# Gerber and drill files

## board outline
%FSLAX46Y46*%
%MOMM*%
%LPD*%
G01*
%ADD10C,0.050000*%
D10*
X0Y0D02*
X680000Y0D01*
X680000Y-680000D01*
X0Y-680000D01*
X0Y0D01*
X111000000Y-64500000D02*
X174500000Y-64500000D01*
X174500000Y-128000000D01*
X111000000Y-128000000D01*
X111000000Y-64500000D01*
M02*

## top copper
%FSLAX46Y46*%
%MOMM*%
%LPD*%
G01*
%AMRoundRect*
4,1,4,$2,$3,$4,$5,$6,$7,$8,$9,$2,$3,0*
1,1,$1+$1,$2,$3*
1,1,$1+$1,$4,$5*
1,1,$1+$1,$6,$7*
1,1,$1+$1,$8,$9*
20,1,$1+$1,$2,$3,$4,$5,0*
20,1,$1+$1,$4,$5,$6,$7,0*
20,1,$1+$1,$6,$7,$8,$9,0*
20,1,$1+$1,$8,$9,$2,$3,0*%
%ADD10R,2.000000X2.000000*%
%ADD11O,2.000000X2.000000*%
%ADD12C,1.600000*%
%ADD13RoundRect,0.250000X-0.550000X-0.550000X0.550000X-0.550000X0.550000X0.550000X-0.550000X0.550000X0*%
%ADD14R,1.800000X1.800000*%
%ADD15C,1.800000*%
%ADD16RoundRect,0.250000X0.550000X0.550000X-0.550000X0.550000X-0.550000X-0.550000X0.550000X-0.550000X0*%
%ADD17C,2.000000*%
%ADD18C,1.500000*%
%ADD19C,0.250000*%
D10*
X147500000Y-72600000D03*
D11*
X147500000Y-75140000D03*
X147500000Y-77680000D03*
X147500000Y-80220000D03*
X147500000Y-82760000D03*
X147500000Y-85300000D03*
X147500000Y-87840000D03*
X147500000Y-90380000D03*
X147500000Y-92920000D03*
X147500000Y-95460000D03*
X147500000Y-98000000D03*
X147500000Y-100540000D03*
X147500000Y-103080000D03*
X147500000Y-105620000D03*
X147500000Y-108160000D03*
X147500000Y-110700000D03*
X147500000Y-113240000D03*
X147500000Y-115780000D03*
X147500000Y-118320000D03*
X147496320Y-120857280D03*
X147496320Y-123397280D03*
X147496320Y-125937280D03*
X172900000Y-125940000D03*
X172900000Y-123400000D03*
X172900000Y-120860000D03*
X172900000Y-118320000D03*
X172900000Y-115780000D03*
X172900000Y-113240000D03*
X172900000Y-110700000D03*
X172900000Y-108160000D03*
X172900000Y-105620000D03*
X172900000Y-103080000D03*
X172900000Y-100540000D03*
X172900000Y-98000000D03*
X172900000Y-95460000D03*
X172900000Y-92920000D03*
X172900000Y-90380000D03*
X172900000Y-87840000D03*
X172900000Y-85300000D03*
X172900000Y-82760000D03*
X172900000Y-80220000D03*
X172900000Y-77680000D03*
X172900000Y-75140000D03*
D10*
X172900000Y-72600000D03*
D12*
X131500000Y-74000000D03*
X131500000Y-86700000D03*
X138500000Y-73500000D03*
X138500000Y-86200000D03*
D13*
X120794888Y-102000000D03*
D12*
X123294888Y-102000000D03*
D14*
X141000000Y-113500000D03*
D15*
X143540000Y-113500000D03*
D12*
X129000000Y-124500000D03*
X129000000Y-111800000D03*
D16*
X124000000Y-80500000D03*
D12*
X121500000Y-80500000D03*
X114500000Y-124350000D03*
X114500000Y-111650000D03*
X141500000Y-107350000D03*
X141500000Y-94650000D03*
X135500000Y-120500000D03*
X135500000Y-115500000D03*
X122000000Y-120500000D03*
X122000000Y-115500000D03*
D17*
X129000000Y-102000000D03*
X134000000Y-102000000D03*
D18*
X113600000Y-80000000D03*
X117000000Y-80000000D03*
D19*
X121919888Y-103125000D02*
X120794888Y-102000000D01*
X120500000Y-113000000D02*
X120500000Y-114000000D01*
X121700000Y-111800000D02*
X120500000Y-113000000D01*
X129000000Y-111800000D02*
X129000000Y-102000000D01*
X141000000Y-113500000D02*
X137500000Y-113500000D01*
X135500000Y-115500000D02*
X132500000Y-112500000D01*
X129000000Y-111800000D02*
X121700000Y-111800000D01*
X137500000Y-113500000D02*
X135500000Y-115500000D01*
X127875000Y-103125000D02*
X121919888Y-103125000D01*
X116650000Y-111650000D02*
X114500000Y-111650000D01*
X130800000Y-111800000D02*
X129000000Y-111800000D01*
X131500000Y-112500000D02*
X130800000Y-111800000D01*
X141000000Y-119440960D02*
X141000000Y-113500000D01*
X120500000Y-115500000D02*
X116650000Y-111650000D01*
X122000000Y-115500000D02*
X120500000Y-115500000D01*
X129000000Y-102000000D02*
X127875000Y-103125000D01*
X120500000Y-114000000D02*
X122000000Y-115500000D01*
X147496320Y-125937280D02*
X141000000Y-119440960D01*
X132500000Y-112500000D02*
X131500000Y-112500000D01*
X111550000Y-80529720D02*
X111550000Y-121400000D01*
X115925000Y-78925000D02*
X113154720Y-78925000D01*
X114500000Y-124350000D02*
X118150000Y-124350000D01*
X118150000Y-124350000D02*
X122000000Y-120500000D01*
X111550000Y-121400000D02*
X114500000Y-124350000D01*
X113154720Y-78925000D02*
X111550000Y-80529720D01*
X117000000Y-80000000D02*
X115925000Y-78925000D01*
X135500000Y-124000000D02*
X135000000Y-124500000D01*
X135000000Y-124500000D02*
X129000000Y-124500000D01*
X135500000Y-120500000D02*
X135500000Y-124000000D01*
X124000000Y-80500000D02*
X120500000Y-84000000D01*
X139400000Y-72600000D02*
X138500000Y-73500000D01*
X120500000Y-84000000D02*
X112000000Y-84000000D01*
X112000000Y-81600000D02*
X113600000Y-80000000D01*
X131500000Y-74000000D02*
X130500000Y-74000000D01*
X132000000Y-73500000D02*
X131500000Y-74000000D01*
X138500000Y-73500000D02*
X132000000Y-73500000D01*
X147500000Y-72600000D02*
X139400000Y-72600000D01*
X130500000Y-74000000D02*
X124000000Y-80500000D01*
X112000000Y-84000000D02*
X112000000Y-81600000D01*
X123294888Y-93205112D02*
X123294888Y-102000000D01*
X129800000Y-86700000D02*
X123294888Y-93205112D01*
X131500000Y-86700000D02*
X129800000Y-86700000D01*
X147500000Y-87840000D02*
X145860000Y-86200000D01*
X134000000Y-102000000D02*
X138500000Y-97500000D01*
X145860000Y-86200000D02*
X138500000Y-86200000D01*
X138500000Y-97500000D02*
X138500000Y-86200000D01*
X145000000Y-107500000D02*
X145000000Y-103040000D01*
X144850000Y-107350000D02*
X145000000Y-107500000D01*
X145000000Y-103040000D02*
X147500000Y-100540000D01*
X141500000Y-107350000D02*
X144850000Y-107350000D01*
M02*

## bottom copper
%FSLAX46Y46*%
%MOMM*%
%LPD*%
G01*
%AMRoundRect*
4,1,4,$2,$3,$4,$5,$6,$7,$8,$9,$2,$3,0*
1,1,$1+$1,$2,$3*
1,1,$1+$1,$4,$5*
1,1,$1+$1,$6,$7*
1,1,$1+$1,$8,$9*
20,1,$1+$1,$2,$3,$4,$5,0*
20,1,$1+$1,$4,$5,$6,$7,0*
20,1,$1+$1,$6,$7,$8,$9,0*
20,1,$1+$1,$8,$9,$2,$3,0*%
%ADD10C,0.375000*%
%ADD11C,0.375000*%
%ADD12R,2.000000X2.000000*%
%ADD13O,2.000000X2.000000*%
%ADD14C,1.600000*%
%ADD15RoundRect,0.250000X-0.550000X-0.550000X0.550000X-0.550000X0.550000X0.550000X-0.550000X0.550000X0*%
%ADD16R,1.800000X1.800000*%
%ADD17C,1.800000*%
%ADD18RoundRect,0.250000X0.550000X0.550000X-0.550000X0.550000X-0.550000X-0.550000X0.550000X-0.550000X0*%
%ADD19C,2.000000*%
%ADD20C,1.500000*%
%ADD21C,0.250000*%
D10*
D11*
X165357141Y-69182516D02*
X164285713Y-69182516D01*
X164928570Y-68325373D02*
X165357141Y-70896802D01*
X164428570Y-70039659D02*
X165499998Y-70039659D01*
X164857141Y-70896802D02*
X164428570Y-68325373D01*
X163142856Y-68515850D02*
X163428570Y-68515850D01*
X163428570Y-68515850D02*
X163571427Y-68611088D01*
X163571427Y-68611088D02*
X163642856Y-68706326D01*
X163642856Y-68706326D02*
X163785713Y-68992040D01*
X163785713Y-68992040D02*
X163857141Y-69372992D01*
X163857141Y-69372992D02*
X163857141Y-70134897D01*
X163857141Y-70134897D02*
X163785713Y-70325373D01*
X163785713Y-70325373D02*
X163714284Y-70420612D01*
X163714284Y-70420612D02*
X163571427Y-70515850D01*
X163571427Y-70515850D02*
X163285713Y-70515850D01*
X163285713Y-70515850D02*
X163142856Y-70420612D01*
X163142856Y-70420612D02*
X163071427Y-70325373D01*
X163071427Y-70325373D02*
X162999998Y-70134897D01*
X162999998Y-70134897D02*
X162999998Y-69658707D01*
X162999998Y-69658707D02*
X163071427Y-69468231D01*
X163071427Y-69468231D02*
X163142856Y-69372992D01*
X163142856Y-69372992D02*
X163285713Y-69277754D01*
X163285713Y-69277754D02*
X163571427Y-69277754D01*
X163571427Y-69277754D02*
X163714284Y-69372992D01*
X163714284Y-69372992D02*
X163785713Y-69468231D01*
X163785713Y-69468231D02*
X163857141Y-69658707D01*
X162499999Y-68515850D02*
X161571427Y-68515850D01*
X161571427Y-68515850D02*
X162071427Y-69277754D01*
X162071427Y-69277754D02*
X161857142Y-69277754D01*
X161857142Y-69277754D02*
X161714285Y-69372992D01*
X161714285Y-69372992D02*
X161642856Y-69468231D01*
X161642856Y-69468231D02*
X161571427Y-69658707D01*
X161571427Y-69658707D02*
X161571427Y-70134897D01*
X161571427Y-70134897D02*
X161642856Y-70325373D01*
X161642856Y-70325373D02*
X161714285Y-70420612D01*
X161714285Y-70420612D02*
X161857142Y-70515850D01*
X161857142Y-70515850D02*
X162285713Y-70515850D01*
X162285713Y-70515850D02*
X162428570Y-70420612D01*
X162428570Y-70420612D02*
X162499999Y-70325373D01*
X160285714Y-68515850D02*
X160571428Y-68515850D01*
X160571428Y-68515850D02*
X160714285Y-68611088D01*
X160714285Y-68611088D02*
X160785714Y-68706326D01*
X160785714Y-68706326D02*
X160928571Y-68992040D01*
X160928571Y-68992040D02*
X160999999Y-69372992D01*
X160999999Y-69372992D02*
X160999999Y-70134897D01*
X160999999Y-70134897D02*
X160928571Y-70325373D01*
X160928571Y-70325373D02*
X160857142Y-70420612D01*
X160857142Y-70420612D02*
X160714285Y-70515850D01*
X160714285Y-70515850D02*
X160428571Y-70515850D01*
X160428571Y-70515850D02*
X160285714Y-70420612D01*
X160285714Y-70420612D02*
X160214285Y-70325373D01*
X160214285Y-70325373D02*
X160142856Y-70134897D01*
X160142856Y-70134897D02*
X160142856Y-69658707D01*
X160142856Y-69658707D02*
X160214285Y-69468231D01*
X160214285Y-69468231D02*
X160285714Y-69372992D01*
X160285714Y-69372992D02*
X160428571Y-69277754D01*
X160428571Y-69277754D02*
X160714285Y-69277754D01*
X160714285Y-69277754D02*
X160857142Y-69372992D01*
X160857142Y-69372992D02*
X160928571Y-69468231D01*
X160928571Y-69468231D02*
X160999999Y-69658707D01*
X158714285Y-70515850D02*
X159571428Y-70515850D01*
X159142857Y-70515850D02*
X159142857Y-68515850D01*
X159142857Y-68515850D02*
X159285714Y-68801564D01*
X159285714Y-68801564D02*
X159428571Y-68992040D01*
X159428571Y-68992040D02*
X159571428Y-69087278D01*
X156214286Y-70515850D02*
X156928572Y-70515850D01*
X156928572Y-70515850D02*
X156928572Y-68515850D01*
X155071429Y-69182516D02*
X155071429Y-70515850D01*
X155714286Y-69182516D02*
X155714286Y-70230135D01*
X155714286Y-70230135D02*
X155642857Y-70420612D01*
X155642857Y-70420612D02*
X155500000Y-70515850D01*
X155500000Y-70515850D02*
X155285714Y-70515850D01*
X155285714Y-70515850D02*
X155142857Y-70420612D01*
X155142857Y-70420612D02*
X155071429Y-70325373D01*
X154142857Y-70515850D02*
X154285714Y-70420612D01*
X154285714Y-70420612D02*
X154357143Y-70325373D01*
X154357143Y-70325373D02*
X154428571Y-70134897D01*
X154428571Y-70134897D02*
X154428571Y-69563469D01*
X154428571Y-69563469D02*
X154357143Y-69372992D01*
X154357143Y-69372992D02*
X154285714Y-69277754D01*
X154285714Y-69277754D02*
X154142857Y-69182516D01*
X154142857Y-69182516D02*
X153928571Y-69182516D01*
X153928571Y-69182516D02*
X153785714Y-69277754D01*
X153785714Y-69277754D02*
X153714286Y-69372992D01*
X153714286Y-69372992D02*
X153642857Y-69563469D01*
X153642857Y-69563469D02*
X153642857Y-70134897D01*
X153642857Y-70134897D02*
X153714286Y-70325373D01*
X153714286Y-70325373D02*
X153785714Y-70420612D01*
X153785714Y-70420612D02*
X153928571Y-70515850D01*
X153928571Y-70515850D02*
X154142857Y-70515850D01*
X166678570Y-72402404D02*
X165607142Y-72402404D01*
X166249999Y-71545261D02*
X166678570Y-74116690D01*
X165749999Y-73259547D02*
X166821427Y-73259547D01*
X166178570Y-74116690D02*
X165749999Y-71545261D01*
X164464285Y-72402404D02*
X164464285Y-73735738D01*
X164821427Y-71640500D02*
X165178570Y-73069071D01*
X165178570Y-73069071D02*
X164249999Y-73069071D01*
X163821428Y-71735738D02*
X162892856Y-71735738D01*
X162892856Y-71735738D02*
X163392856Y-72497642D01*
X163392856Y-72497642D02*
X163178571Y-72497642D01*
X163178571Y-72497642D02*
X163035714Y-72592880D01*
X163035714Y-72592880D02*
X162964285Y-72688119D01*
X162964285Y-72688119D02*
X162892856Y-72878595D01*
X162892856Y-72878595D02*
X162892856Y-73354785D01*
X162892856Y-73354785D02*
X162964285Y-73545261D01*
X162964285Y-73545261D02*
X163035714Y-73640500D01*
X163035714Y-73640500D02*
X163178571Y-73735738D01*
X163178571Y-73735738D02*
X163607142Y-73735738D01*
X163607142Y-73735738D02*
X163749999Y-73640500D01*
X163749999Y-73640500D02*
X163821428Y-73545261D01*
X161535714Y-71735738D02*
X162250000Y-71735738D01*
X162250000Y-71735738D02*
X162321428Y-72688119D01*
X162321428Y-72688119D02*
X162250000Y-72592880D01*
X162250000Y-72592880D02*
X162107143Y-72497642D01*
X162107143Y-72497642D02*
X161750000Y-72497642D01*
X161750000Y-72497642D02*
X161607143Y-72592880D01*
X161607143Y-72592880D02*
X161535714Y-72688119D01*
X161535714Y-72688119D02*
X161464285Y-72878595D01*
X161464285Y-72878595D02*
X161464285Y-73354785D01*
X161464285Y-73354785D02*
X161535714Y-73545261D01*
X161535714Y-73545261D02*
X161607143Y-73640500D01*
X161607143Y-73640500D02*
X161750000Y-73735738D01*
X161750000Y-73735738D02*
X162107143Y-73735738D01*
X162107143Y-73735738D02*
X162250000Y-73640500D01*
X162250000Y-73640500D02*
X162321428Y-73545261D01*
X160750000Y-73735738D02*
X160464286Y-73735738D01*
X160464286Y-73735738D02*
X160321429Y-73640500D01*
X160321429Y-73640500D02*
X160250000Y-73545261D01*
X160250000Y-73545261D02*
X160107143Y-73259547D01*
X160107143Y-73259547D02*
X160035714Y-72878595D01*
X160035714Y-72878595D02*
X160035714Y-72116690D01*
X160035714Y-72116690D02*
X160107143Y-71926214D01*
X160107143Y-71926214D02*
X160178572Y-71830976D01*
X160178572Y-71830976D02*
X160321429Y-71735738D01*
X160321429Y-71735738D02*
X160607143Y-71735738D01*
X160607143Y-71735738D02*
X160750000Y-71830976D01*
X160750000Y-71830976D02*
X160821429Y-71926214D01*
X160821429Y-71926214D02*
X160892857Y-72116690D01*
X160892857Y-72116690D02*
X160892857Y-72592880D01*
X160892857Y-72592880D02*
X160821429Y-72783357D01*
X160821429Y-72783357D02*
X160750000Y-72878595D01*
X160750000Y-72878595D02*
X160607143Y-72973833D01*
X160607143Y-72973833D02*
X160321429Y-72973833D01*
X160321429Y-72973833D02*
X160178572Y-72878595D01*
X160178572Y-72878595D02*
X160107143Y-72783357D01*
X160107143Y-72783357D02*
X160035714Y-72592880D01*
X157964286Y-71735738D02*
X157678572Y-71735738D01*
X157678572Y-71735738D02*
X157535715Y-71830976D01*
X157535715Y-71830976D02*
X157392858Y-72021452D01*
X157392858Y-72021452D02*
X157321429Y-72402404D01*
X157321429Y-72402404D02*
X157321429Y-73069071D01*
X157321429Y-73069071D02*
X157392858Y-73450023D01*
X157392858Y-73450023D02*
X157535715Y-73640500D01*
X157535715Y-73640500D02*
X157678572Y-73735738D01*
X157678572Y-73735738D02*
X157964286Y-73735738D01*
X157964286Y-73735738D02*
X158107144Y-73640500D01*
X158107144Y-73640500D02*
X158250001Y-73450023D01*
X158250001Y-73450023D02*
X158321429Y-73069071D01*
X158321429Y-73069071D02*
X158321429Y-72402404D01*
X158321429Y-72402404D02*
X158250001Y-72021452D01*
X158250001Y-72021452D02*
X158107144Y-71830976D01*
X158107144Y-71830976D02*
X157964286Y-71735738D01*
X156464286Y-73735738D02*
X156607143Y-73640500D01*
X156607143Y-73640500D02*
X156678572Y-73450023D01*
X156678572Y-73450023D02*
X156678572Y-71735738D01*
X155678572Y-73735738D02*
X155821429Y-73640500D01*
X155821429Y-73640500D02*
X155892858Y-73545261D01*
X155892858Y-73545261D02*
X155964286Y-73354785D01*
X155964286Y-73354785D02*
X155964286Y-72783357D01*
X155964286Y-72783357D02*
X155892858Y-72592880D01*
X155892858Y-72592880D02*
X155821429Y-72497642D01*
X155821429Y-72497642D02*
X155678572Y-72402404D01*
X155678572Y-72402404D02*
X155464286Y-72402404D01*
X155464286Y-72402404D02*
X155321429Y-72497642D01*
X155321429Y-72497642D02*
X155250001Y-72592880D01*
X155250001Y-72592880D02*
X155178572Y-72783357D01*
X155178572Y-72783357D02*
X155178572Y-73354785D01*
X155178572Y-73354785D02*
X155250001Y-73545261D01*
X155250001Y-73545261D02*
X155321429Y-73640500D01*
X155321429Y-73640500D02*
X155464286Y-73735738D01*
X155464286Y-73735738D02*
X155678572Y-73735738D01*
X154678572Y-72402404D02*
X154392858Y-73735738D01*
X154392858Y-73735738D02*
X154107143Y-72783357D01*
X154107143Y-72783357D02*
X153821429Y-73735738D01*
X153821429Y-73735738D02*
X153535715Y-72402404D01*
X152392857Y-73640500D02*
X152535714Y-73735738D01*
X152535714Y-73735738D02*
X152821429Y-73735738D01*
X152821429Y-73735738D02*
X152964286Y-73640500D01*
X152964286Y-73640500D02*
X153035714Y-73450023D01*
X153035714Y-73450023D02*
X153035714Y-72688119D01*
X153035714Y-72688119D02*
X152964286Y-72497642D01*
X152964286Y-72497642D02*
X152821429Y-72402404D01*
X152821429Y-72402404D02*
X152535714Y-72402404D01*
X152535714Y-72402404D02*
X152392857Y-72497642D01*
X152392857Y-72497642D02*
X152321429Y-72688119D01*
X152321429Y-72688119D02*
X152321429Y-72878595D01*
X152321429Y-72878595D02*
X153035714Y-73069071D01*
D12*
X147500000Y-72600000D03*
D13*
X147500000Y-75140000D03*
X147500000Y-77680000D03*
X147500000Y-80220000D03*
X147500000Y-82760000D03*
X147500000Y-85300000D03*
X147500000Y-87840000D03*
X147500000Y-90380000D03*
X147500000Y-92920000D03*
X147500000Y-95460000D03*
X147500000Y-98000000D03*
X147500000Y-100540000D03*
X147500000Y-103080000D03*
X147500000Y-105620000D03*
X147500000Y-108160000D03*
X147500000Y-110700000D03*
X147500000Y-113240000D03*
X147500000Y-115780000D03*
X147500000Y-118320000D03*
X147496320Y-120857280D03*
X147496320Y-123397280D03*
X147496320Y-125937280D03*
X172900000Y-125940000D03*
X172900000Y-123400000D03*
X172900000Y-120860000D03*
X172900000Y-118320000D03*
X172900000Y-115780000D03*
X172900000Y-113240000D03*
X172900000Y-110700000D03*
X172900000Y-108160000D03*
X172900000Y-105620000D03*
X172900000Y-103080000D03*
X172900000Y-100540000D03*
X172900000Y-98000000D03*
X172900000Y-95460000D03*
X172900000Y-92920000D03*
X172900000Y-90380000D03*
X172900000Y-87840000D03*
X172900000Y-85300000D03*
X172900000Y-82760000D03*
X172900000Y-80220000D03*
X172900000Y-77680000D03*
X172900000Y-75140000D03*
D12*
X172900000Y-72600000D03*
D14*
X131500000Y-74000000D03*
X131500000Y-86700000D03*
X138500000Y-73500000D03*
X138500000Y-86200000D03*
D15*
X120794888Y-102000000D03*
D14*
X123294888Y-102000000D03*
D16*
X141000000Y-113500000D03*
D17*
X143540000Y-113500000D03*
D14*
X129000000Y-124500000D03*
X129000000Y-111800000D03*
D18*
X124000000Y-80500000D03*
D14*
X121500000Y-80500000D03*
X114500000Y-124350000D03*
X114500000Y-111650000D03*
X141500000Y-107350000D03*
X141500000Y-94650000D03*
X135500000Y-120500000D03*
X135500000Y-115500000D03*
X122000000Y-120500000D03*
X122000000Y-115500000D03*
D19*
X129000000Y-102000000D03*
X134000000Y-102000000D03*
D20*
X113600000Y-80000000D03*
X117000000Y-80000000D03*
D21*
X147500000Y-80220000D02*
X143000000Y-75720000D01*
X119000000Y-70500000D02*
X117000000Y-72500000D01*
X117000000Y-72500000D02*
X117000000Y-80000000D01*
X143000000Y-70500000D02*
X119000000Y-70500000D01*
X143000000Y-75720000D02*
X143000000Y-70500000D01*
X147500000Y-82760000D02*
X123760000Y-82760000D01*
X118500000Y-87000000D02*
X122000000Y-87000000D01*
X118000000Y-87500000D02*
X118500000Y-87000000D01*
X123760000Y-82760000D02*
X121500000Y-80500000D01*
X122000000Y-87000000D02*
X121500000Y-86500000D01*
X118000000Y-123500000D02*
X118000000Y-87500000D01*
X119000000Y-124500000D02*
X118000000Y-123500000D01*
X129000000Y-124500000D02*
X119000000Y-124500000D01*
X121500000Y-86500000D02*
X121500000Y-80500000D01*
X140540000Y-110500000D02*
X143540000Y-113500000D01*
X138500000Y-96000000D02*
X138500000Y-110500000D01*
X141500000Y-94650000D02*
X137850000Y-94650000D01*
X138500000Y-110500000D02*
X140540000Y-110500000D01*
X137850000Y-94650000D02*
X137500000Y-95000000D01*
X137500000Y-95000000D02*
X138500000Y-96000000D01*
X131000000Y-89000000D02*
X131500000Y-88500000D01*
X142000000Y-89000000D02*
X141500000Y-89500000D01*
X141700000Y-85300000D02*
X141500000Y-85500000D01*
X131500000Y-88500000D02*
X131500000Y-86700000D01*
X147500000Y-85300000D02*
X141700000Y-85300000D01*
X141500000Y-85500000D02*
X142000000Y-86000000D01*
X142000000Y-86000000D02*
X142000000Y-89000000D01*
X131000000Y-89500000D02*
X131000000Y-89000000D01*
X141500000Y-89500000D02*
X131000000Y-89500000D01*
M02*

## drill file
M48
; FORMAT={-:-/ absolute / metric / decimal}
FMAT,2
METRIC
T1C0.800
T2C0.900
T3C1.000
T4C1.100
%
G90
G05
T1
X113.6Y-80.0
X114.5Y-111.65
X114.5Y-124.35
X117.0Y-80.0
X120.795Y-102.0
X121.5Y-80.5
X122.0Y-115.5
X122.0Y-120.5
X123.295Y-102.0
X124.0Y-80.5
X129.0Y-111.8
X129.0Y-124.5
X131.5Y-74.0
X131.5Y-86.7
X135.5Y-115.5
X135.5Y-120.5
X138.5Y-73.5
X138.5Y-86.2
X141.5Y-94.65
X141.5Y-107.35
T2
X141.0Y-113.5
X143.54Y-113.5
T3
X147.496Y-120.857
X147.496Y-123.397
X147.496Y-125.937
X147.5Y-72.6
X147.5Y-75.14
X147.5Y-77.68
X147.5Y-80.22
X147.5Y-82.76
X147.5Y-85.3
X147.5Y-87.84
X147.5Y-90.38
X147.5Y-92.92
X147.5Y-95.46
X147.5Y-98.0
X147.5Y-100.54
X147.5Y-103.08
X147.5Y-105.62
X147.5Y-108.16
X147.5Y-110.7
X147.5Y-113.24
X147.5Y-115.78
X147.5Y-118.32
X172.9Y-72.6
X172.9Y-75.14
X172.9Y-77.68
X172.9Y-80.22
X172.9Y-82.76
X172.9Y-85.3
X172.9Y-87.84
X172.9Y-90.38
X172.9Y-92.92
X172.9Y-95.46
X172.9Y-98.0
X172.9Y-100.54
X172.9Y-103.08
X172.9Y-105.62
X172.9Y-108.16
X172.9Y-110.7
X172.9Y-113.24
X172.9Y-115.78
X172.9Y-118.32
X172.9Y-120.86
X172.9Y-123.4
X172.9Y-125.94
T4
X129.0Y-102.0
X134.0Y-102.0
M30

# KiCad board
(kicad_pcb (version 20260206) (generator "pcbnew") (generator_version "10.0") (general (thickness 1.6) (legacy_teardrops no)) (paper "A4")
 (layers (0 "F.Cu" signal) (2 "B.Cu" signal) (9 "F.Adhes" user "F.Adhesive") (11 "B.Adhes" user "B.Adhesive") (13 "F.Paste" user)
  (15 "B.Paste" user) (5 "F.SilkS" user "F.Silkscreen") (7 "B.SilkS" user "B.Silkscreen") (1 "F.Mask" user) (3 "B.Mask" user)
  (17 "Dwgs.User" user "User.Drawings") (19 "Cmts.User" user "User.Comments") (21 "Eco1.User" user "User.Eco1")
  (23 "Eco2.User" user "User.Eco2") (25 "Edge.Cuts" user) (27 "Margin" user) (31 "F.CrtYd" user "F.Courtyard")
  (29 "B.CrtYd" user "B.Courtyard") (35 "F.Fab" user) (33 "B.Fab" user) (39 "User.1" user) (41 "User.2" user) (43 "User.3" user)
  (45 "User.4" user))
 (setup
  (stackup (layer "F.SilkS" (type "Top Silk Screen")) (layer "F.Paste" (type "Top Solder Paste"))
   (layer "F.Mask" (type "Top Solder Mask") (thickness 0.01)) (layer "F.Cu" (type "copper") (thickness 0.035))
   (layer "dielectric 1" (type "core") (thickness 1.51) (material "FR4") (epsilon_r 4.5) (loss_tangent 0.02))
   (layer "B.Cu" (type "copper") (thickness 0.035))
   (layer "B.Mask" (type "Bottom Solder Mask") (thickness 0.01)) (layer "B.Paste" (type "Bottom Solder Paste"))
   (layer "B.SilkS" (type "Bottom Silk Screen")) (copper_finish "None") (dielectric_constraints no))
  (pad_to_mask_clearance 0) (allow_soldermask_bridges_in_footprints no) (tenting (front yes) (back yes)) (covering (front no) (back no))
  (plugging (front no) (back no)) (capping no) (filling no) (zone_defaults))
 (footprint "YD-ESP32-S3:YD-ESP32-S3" (layer "F.Cu") (at 146.2 70.69)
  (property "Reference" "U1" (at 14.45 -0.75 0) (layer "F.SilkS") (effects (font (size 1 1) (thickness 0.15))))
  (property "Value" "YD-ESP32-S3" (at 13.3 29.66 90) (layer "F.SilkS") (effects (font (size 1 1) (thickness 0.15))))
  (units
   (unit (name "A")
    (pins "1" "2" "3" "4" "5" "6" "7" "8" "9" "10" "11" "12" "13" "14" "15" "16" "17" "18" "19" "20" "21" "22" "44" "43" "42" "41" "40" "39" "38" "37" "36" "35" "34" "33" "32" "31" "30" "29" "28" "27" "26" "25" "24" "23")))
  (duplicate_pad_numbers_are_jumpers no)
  (pad "1" thru_hole rect (at 1.3 1.91 270) (size 2 2) (drill 1) (layers "*.Cu" "*.Mask") (remove_unused_layers no) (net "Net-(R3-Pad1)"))
  (pad "2" thru_hole oval (at 1.3 4.45 270) (size 2 2) (drill 1) (layers "*.Cu" "*.Mask") (remove_unused_layers no)
   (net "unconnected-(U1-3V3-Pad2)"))
  (pad "3" thru_hole oval (at 1.3 6.99 270) (size 2 2) (drill 1) (layers "*.Cu" "*.Mask") (remove_unused_layers no)
   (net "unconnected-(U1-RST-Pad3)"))
  (pad "4" thru_hole oval (at 1.3 9.53 270) (size 2 2) (drill 1) (layers "*.Cu" "*.Mask") (remove_unused_layers no) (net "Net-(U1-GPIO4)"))
  (pad "5" thru_hole oval (at 1.3 12.07 270) (size 2 2) (drill 1) (layers "*.Cu" "*.Mask") (remove_unused_layers no) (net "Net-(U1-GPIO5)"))
  (pad "6" thru_hole oval (at 1.3 14.61 270) (size 2 2) (drill 1) (layers "*.Cu" "*.Mask") (remove_unused_layers no) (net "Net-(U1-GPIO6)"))
  (pad "7" thru_hole oval (at 1.3 17.15 270) (size 2 2) (drill 1) (layers "*.Cu" "*.Mask") (remove_unused_layers no) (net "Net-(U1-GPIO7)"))
  (pad "8" thru_hole oval (at 1.3 19.69 270) (size 2 2) (drill 1) (layers "*.Cu" "*.Mask") (remove_unused_layers no)
   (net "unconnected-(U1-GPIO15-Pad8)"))
  (pad "9" thru_hole oval (at 1.3 22.23 270) (size 2 2) (drill 1) (layers "*.Cu" "*.Mask") (remove_unused_layers no)
   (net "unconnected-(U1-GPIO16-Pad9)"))
  (pad "10" thru_hole oval (at 1.3 24.77 270) (size 2 2) (drill 1) (layers "*.Cu" "*.Mask") (remove_unused_layers no)
   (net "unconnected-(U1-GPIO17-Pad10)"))
  (pad "11" thru_hole oval (at 1.3 27.31 270) (size 2 2) (drill 1) (layers "*.Cu" "*.Mask") (remove_unused_layers no)
   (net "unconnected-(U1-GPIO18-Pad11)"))
  (pad "12" thru_hole oval (at 1.3 29.85 270) (size 2 2) (drill 1) (layers "*.Cu" "*.Mask") (remove_unused_layers no) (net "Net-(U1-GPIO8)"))
  (pad "13" thru_hole oval (at 1.3 32.39 270) (size 2 2) (drill 1) (layers "*.Cu" "*.Mask") (remove_unused_layers no)
   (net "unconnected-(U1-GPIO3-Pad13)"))
  (pad "14" thru_hole oval (at 1.3 34.93 270) (size 2 2) (drill 1) (layers "*.Cu" "*.Mask") (remove_unused_layers no)
   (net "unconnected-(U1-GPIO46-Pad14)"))
  (pad "15" thru_hole oval (at 1.3 37.47 270) (size 2 2) (drill 1) (layers "*.Cu" "*.Mask") (remove_unused_layers no)
   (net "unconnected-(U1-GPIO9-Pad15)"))
  (pad "16" thru_hole oval (at 1.3 40.01 270) (size 2 2) (drill 1) (layers "*.Cu" "*.Mask") (remove_unused_layers no)
   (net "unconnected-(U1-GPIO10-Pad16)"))
  (pad "17" thru_hole oval (at 1.3 42.55 270) (size 2 2) (drill 1) (layers "*.Cu" "*.Mask") (remove_unused_layers no)
   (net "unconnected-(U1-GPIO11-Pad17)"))
  (pad "18" thru_hole oval (at 1.3 45.09 270) (size 2 2) (drill 1) (layers "*.Cu" "*.Mask") (remove_unused_layers no)
   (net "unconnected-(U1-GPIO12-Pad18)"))
  (pad "19" thru_hole oval (at 1.3 47.63 270) (size 2 2) (drill 1) (layers "*.Cu" "*.Mask") (remove_unused_layers no)
   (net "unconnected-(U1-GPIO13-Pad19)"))
  (pad "20" thru_hole oval (at 1.29632 50.16728 270) (size 2 2) (drill 1) (layers "*.Cu" "*.Mask") (remove_unused_layers no)
   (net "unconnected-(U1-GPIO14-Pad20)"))
  (pad "21" thru_hole oval (at 1.29632 52.70728 270) (size 2 2) (drill 1) (layers "*.Cu" "*.Mask") (remove_unused_layers no)
   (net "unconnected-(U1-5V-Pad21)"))
  (pad "22" thru_hole oval (at 1.29632 55.24728 270) (size 2 2) (drill 1) (layers "*.Cu" "*.Mask") (remove_unused_layers no) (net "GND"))
  (pad "23" thru_hole oval (at 26.7 55.25 270) (size 2 2) (drill 1) (layers "*.Cu" "*.Mask") (remove_unused_layers no)
   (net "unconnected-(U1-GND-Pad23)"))
  (pad "24" thru_hole oval (at 26.7 52.71 270) (size 2 2) (drill 1) (layers "*.Cu" "*.Mask") (remove_unused_layers no)
   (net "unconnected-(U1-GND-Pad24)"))
  (pad "25" thru_hole oval (at 26.7 50.17 270) (size 2 2) (drill 1) (layers "*.Cu" "*.Mask") (remove_unused_layers no)
   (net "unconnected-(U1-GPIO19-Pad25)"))
  (pad "26" thru_hole oval (at 26.7 47.63 270) (size 2 2) (drill 1) (layers "*.Cu" "*.Mask") (remove_unused_layers no)
   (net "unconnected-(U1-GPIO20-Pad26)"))
  (pad "27" thru_hole oval (at 26.7 45.09 270) (size 2 2) (drill 1) (layers "*.Cu" "*.Mask") (remove_unused_layers no)
   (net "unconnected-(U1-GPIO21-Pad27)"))
  (pad "28" thru_hole oval (at 26.7 42.55 270) (size 2 2) (drill 1) (layers "*.Cu" "*.Mask") (remove_unused_layers no)
   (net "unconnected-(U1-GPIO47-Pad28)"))
  (pad "29" thru_hole oval (at 26.7 40.01 270) (size 2 2) (drill 1) (layers "*.Cu" "*.Mask") (remove_unused_layers no)
   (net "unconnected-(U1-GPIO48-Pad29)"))
  (pad "30" thru_hole oval (at 26.7 37.47 270) (size 2 2) (drill 1) (layers "*.Cu" "*.Mask") (remove_unused_layers no)
   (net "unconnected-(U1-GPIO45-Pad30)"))
  (pad "31" thru_hole oval (at 26.7 34.93 270) (size 2 2) (drill 1) (layers "*.Cu" "*.Mask") (remove_unused_layers no)
   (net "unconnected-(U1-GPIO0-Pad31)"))
  (pad "32" thru_hole oval (at 26.7 32.39 270) (size 2 2) (drill 1) (layers "*.Cu" "*.Mask") (remove_unused_layers no)
   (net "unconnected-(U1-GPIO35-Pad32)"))
  (pad "33" thru_hole oval (at 26.7 29.85 270) (size 2 2) (drill 1) (layers "*.Cu" "*.Mask") (remove_unused_layers no)
   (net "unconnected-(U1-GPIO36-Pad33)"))
  (pad "34" thru_hole oval (at 26.7 27.31 270) (size 2 2) (drill 1) (layers "*.Cu" "*.Mask") (remove_unused_layers no)
   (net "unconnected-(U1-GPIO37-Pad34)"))
  (pad "35" thru_hole oval (at 26.7 24.77 270) (size 2 2) (drill 1) (layers "*.Cu" "*.Mask") (remove_unused_layers no)
   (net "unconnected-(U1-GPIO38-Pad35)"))
  (pad "36" thru_hole oval (at 26.7 22.23 270) (size 2 2) (drill 1) (layers "*.Cu" "*.Mask") (remove_unused_layers no)
   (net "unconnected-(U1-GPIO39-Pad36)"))
  (pad "37" thru_hole oval (at 26.7 19.69 270) (size 2 2) (drill 1) (layers "*.Cu" "*.Mask") (remove_unused_layers no)
   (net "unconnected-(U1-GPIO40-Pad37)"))
  (pad "38" thru_hole oval (at 26.7 17.15 270) (size 2 2) (drill 1) (layers "*.Cu" "*.Mask") (remove_unused_layers no)
   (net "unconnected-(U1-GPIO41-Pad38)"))
  (pad "39" thru_hole oval (at 26.7 14.61 270) (size 2 2) (drill 1) (layers "*.Cu" "*.Mask") (remove_unused_layers no)
   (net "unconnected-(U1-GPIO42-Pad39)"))
  (pad "40" thru_hole oval (at 26.7 12.07 270) (size 2 2) (drill 1) (layers "*.Cu" "*.Mask") (remove_unused_layers no)
   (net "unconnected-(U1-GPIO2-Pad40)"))
  (pad "41" thru_hole oval (at 26.7 9.53 270) (size 2 2) (drill 1) (layers "*.Cu" "*.Mask") (remove_unused_layers no)
   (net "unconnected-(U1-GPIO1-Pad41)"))
  (pad "42" thru_hole oval (at 26.7 6.99 270) (size 2 2) (drill 1) (layers "*.Cu" "*.Mask") (remove_unused_layers no)
   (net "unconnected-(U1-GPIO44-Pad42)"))
  (pad "43" thru_hole oval (at 26.7 4.45 270) (size 2 2) (drill 1) (layers "*.Cu" "*.Mask") (remove_unused_layers no)
   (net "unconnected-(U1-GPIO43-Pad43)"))
  (pad "44" thru_hole rect (at 26.7 1.91 270) (size 2 2) (drill 1) (layers "*.Cu" "*.Mask") (remove_unused_layers no)
   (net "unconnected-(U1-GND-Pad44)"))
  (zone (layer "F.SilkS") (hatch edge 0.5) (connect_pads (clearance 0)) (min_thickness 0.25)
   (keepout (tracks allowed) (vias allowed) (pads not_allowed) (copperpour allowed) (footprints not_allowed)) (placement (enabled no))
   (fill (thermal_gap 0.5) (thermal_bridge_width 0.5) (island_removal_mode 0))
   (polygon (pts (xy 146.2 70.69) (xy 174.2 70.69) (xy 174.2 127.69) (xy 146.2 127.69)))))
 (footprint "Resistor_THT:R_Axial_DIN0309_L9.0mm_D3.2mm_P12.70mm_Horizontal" (layer "F.Cu") (at 131.5 74 -90)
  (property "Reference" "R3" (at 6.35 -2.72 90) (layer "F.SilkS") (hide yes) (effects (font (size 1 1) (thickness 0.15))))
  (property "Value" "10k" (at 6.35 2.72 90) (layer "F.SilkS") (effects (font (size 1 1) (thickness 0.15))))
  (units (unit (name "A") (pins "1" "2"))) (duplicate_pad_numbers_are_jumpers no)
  (pad "1" thru_hole circle (at 0 0 270) (size 1.6 1.6) (drill 0.8) (layers "*.Cu" "*.Mask") (remove_unused_layers no) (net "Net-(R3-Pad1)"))
  (pad "2" thru_hole circle (at 12.7 0 270) (size 1.6 1.6) (drill 0.8) (layers "*.Cu" "*.Mask") (remove_unused_layers no)
   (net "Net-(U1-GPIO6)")))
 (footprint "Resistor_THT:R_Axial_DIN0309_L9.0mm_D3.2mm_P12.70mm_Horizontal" (layer "F.Cu") (at 138.5 73.5 -90)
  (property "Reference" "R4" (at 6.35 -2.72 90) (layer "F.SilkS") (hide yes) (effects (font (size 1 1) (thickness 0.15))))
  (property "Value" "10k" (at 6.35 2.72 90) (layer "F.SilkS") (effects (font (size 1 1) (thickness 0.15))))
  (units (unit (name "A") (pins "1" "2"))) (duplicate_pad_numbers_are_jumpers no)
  (pad "1" thru_hole circle (at 0 0 270) (size 1.6 1.6) (drill 0.8) (layers "*.Cu" "*.Mask") (remove_unused_layers no) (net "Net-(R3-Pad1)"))
  (pad "2" thru_hole circle (at 12.7 0 270) (size 1.6 1.6) (drill 0.8) (layers "*.Cu" "*.Mask") (remove_unused_layers no)
   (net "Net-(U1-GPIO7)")))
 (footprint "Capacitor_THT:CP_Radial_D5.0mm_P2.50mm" (layer "F.Cu") (at 120.794888 102)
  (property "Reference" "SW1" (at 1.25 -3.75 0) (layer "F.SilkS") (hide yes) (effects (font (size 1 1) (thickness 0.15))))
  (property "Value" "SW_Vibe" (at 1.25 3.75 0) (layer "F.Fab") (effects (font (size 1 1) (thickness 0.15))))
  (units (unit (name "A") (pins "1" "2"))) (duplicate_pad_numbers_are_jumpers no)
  (pad "1" thru_hole roundrect (at 0 0) (size 1.6 1.6) (drill 0.8) (layers "*.Cu" "*.Mask") (remove_unused_layers no)
   (roundrect_rratio 0.15625) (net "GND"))
  (pad "2" thru_hole circle (at 2.5 0) (size 1.6 1.6) (drill 0.8) (layers "*.Cu" "*.Mask") (remove_unused_layers no) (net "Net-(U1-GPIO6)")))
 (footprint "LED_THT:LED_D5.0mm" (layer "F.Cu") (at 141 113.5)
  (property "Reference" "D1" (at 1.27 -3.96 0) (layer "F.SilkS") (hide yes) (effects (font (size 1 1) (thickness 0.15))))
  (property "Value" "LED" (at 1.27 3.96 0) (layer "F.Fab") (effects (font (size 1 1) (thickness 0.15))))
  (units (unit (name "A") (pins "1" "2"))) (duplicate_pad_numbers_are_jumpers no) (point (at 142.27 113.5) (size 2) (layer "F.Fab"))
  (pad "1" thru_hole rect (at 0 0) (size 1.8 1.8) (drill 0.9) (layers "*.Cu" "*.Mask") (remove_unused_layers no) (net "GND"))
  (pad "2" thru_hole circle (at 2.54 0) (size 1.8 1.8) (drill 0.9) (layers "*.Cu" "*.Mask") (remove_unused_layers no) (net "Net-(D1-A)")))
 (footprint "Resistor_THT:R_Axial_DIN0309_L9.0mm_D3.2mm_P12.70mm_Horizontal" (layer "F.Cu") (at 129 124.5 90)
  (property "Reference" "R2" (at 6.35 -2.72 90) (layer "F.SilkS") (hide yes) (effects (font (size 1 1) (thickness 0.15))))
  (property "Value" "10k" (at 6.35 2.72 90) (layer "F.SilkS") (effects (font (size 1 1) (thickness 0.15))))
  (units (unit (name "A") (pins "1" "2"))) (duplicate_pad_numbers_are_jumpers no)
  (pad "1" thru_hole circle (at 0 0 90) (size 1.6 1.6) (drill 0.8) (layers "*.Cu" "*.Mask") (remove_unused_layers no) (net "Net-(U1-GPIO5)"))
  (pad "2" thru_hole circle (at 12.7 0 90) (size 1.6 1.6) (drill 0.8) (layers "*.Cu" "*.Mask") (remove_unused_layers no) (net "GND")))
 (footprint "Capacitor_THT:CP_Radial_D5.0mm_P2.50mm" (layer "F.Cu") (at 124 80.5 180)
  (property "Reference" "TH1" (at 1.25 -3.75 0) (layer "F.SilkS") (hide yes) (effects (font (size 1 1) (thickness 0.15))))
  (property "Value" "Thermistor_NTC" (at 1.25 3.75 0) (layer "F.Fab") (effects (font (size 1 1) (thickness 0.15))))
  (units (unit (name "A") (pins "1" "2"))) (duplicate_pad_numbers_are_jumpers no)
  (pad "1" thru_hole roundrect (at 0 0 180) (size 1.6 1.6) (drill 0.8) (layers "*.Cu" "*.Mask") (remove_unused_layers no)
   (roundrect_rratio 0.15625) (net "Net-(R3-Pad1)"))
  (pad "2" thru_hole circle (at 2.5 0 180) (size 1.6 1.6) (drill 0.8) (layers "*.Cu" "*.Mask") (remove_unused_layers no)
   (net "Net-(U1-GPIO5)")))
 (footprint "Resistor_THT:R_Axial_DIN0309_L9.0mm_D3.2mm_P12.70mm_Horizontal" (layer "F.Cu") (at 114.5 124.35 90)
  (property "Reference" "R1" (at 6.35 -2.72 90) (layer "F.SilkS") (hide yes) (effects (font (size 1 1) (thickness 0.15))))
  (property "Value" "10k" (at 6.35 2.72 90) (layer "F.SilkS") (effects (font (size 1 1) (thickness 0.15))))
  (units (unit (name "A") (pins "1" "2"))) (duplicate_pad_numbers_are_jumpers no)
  (pad "1" thru_hole circle (at 0 0 90) (size 1.6 1.6) (drill 0.8) (layers "*.Cu" "*.Mask") (remove_unused_layers no) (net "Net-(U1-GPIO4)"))
  (pad "2" thru_hole circle (at 12.7 0 90) (size 1.6 1.6) (drill 0.8) (layers "*.Cu" "*.Mask") (remove_unused_layers no) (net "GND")))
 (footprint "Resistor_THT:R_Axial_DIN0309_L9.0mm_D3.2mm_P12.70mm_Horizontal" (layer "F.Cu") (at 141.5 107.35 90)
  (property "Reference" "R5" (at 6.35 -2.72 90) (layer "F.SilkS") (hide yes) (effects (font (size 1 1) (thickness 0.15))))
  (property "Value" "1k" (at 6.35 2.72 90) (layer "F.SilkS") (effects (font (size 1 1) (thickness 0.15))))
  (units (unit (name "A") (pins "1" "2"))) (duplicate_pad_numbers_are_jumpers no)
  (pad "1" thru_hole circle (at 0 0 90) (size 1.6 1.6) (drill 0.8) (layers "*.Cu" "*.Mask") (remove_unused_layers no) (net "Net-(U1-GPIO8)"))
  (pad "2" thru_hole circle (at 12.7 0 90) (size 1.6 1.6) (drill 0.8) (layers "*.Cu" "*.Mask") (remove_unused_layers no) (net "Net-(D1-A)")))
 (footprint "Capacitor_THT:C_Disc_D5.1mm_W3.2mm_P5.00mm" (layer "F.Cu") (at 135.5 120.5 90)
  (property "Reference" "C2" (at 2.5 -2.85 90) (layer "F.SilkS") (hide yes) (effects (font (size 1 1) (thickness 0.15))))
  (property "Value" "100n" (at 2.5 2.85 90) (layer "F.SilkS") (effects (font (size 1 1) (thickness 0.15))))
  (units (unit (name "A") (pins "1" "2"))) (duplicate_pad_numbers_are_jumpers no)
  (pad "1" thru_hole circle (at 0 0 90) (size 1.6 1.6) (drill 0.8) (layers "*.Cu" "*.Mask") (remove_unused_layers no) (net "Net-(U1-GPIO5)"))
  (pad "2" thru_hole circle (at 5 0 90) (size 1.6 1.6) (drill 0.8) (layers "*.Cu" "*.Mask") (remove_unused_layers no) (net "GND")))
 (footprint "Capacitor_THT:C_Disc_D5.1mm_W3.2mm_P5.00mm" (layer "F.Cu") (at 122 120.5 90)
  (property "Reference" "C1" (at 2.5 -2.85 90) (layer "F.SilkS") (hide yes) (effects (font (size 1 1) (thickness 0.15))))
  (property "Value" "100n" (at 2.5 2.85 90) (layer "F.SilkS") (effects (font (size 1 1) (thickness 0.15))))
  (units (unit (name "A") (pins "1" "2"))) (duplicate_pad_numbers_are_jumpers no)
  (pad "1" thru_hole circle (at 0 0 90) (size 1.6 1.6) (drill 0.8) (layers "*.Cu" "*.Mask") (remove_unused_layers no) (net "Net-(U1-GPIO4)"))
  (pad "2" thru_hole circle (at 5 0 90) (size 1.6 1.6) (drill 0.8) (layers "*.Cu" "*.Mask") (remove_unused_layers no) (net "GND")))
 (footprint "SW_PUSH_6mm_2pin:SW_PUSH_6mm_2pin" (layer "F.Cu") (at 131.5 102)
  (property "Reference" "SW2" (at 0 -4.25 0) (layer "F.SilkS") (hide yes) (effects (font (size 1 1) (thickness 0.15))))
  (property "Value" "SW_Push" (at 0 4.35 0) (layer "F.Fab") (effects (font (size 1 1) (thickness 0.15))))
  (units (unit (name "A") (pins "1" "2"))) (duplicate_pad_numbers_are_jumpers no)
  (pad "1" thru_hole circle (at -2.5 0 90) (size 2 2) (drill 1.1) (layers "*.Cu" "*.Mask") (remove_unused_layers no) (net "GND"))
  (pad "2" thru_hole circle (at 2.5 0 90) (size 2 2) (drill 1.1) (layers "*.Cu" "*.Mask") (remove_unused_layers no) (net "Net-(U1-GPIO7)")))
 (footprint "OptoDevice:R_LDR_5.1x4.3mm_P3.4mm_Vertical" (layer "F.Cu") (at 113.6 80)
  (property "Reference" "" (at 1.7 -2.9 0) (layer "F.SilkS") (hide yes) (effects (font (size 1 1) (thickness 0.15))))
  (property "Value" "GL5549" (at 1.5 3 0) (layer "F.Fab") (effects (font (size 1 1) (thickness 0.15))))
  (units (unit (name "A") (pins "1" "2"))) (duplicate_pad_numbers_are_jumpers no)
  (pad "1" thru_hole circle (at 0 0) (size 1.5 1.5) (drill 0.8) (layers "*.Cu" "*.Mask") (remove_unused_layers no) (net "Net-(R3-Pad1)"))
  (pad "2" thru_hole circle (at 3.4 0) (size 1.5 1.5) (drill 0.8) (layers "*.Cu" "*.Mask") (remove_unused_layers no) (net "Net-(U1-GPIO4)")))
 (gr_rect (start 0 0) (end 0.68 0.68) (stroke (width 0.05) (type solid)) (fill no) (layer "Edge.Cuts"))
 (gr_rect (start 111 64.5) (end 174.5 128) (stroke (width 0.05) (type default)) (fill no) (layer "Edge.Cuts"))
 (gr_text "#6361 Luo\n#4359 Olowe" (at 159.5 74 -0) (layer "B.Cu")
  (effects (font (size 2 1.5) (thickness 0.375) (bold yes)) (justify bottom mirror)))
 (segment (start 121.919888 103.125) (end 120.794888 102) (width 0.25) (layer "F.Cu") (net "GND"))
 (segment (start 120.5 113) (end 120.5 114) (width 0.25) (layer "F.Cu") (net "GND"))
 (segment (start 121.7 111.8) (end 120.5 113) (width 0.25) (layer "F.Cu") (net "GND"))
 (segment (start 129 111.8) (end 129 102) (width 0.25) (layer "F.Cu") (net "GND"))
 (segment (start 141 113.5) (end 137.5 113.5) (width 0.25) (layer "F.Cu") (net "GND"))
 (segment (start 135.5 115.5) (end 132.5 112.5) (width 0.25) (layer "F.Cu") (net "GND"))
 (segment (start 129 111.8) (end 121.7 111.8) (width 0.25) (layer "F.Cu") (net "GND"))
 (segment (start 137.5 113.5) (end 135.5 115.5) (width 0.25) (layer "F.Cu") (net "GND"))
 (segment (start 127.875 103.125) (end 121.919888 103.125) (width 0.25) (layer "F.Cu") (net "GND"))
 (segment (start 116.65 111.65) (end 114.5 111.65) (width 0.25) (layer "F.Cu") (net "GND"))
 (segment (start 130.8 111.8) (end 129 111.8) (width 0.25) (layer "F.Cu") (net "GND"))
 (segment (start 131.5 112.5) (end 130.8 111.8) (width 0.25) (layer "F.Cu") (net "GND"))
 (segment (start 141 119.44096) (end 141 113.5) (width 0.25) (layer "F.Cu") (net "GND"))
 (segment (start 120.5 115.5) (end 116.65 111.65) (width 0.25) (layer "F.Cu") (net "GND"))
 (segment (start 122 115.5) (end 120.5 115.5) (width 0.25) (layer "F.Cu") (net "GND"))
 (segment (start 129 102) (end 127.875 103.125) (width 0.25) (layer "F.Cu") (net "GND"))
 (segment (start 120.5 114) (end 122 115.5) (width 0.25) (layer "F.Cu") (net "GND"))
 (segment (start 147.49632 125.93728) (end 141 119.44096) (width 0.25) (layer "F.Cu") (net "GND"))
 (segment (start 132.5 112.5) (end 131.5 112.5) (width 0.25) (layer "F.Cu") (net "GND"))
 (segment (start 111.55 80.52972) (end 111.55 121.4) (width 0.25) (layer "F.Cu") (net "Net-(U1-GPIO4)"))
 (segment (start 115.925 78.925) (end 113.15472 78.925) (width 0.25) (layer "F.Cu") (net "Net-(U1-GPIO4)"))
 (segment (start 114.5 124.35) (end 118.15 124.35) (width 0.25) (layer "F.Cu") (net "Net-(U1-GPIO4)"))
 (segment (start 118.15 124.35) (end 122 120.5) (width 0.25) (layer "F.Cu") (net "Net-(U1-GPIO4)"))
 (segment (start 111.55 121.4) (end 114.5 124.35) (width 0.25) (layer "F.Cu") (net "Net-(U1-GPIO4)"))
 (segment (start 113.15472 78.925) (end 111.55 80.52972) (width 0.25) (layer "F.Cu") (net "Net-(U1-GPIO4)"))
 (segment (start 117 80) (end 115.925 78.925) (width 0.25) (layer "F.Cu") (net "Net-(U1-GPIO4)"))
 (segment (start 147.5 80.22) (end 143 75.72) (width 0.25) (layer "B.Cu") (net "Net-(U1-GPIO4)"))
 (segment (start 119 70.5) (end 117 72.5) (width 0.25) (layer "B.Cu") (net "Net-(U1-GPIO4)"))
 (segment (start 117 72.5) (end 117 80) (width 0.25) (layer "B.Cu") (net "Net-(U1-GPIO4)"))
 (segment (start 143 70.5) (end 119 70.5) (width 0.25) (layer "B.Cu") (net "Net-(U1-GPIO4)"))
 (segment (start 143 75.72) (end 143 70.5) (width 0.25) (layer "B.Cu") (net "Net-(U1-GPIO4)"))
 (segment (start 135.5 124) (end 135 124.5) (width 0.25) (layer "F.Cu") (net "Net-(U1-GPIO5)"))
 (segment (start 135 124.5) (end 129 124.5) (width 0.25) (layer "F.Cu") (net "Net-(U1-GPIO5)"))
 (segment (start 135.5 120.5) (end 135.5 124) (width 0.25) (layer "F.Cu") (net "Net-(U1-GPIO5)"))
 (segment (start 147.5 82.76) (end 123.76 82.76) (width 0.25) (layer "B.Cu") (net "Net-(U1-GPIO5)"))
 (segment (start 118.5 87) (end 122 87) (width 0.25) (layer "B.Cu") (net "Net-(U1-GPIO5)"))
 (segment (start 118 87.5) (end 118.5 87) (width 0.25) (layer "B.Cu") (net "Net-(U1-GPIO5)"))
 (segment (start 123.76 82.76) (end 121.5 80.5) (width 0.25) (layer "B.Cu") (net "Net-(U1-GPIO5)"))
 (segment (start 122 87) (end 121.5 86.5) (width 0.25) (layer "B.Cu") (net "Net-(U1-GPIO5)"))
 (segment (start 118 123.5) (end 118 87.5) (width 0.25) (layer "B.Cu") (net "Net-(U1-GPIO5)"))
 (segment (start 119 124.5) (end 118 123.5) (width 0.25) (layer "B.Cu") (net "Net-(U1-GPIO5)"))
 (segment (start 129 124.5) (end 119 124.5) (width 0.25) (layer "B.Cu") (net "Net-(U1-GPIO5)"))
 (segment (start 121.5 86.5) (end 121.5 80.5) (width 0.25) (layer "B.Cu") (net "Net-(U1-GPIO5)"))
 (segment (start 140.54 110.5) (end 143.54 113.5) (width 0.25) (layer "B.Cu") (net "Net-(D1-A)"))
 (segment (start 138.5 96) (end 138.5 110.5) (width 0.25) (layer "B.Cu") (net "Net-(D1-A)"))
 (segment (start 141.5 94.65) (end 137.85 94.65) (width 0.25) (layer "B.Cu") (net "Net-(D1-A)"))
 (segment (start 138.5 110.5) (end 140.54 110.5) (width 0.25) (layer "B.Cu") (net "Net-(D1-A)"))
 (segment (start 137.85 94.65) (end 137.5 95) (width 0.25) (layer "B.Cu") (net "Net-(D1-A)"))
 (segment (start 137.5 95) (end 138.5 96) (width 0.25) (layer "B.Cu") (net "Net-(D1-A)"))
 (segment (start 124 80.5) (end 120.5 84) (width 0.25) (layer "F.Cu") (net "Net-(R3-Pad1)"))
 (segment (start 139.4 72.6) (end 138.5 73.5) (width 0.25) (layer "F.Cu") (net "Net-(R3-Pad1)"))
 (segment (start 120.5 84) (end 112 84) (width 0.25) (layer "F.Cu") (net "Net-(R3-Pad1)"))
 (segment (start 112 81.6) (end 113.6 80) (width 0.25) (layer "F.Cu") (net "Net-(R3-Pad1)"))
 (segment (start 131.5 74) (end 130.5 74) (width 0.25) (layer "F.Cu") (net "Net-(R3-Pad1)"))
 (segment (start 132 73.5) (end 131.5 74) (width 0.25) (layer "F.Cu") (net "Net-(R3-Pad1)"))
 (segment (start 138.5 73.5) (end 132 73.5) (width 0.25) (layer "F.Cu") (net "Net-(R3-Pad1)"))
 (segment (start 147.5 72.6) (end 139.4 72.6) (width 0.25) (layer "F.Cu") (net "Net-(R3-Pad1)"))
 (segment (start 130.5 74) (end 124 80.5) (width 0.25) (layer "F.Cu") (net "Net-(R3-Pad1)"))
 (segment (start 112 84) (end 112 81.6) (width 0.25) (layer "F.Cu") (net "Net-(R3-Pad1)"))
 (segment (start 123.294888 93.205112) (end 123.294888 102) (width 0.25) (layer "F.Cu") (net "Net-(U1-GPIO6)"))
 (segment (start 129.8 86.7) (end 123.294888 93.205112) (width 0.25) (layer "F.Cu") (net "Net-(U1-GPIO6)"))
 (segment (start 131.5 86.7) (end 129.8 86.7) (width 0.25) (layer "F.Cu") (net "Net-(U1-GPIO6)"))
 (segment (start 131 89) (end 131.5 88.5) (width 0.25) (layer "B.Cu") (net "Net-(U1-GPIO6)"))
 (segment (start 142 89) (end 141.5 89.5) (width 0.25) (layer "B.Cu") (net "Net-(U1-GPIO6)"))
 (segment (start 141.7 85.3) (end 141.5 85.5) (width 0.25) (layer "B.Cu") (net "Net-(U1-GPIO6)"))
 (segment (start 131.5 88.5) (end 131.5 86.7) (width 0.25) (layer "B.Cu") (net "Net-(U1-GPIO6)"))
 (segment (start 147.5 85.3) (end 141.7 85.3) (width 0.25) (layer "B.Cu") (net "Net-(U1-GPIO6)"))
 (segment (start 141.5 85.5) (end 142 86) (width 0.25) (layer "B.Cu") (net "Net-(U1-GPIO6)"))
 (segment (start 142 86) (end 142 89) (width 0.25) (layer "B.Cu") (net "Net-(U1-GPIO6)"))
 (segment (start 131 89.5) (end 131 89) (width 0.25) (layer "B.Cu") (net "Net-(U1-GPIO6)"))
 (segment (start 141.5 89.5) (end 131 89.5) (width 0.25) (layer "B.Cu") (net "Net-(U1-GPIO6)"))
 (segment (start 147.5 87.84) (end 145.86 86.2) (width 0.25) (layer "F.Cu") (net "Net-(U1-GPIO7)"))
 (segment (start 134 102) (end 138.5 97.5) (width 0.25) (layer "F.Cu") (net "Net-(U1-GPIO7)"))
 (segment (start 145.86 86.2) (end 138.5 86.2) (width 0.25) (layer "F.Cu") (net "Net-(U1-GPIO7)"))
 (segment (start 138.5 97.5) (end 138.5 86.2) (width 0.25) (layer "F.Cu") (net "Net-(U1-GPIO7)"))
 (segment (start 145 107.5) (end 145 103.04) (width 0.25) (layer "F.Cu") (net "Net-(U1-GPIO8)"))
 (segment (start 144.85 107.35) (end 145 107.5) (width 0.25) (layer "F.Cu") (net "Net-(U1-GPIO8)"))
 (segment (start 145 103.04) (end 147.5 100.54) (width 0.25) (layer "F.Cu") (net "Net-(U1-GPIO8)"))
 (segment (start 141.5 107.35) (end 144.85 107.35) (width 0.25) (layer "F.Cu") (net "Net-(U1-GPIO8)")))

